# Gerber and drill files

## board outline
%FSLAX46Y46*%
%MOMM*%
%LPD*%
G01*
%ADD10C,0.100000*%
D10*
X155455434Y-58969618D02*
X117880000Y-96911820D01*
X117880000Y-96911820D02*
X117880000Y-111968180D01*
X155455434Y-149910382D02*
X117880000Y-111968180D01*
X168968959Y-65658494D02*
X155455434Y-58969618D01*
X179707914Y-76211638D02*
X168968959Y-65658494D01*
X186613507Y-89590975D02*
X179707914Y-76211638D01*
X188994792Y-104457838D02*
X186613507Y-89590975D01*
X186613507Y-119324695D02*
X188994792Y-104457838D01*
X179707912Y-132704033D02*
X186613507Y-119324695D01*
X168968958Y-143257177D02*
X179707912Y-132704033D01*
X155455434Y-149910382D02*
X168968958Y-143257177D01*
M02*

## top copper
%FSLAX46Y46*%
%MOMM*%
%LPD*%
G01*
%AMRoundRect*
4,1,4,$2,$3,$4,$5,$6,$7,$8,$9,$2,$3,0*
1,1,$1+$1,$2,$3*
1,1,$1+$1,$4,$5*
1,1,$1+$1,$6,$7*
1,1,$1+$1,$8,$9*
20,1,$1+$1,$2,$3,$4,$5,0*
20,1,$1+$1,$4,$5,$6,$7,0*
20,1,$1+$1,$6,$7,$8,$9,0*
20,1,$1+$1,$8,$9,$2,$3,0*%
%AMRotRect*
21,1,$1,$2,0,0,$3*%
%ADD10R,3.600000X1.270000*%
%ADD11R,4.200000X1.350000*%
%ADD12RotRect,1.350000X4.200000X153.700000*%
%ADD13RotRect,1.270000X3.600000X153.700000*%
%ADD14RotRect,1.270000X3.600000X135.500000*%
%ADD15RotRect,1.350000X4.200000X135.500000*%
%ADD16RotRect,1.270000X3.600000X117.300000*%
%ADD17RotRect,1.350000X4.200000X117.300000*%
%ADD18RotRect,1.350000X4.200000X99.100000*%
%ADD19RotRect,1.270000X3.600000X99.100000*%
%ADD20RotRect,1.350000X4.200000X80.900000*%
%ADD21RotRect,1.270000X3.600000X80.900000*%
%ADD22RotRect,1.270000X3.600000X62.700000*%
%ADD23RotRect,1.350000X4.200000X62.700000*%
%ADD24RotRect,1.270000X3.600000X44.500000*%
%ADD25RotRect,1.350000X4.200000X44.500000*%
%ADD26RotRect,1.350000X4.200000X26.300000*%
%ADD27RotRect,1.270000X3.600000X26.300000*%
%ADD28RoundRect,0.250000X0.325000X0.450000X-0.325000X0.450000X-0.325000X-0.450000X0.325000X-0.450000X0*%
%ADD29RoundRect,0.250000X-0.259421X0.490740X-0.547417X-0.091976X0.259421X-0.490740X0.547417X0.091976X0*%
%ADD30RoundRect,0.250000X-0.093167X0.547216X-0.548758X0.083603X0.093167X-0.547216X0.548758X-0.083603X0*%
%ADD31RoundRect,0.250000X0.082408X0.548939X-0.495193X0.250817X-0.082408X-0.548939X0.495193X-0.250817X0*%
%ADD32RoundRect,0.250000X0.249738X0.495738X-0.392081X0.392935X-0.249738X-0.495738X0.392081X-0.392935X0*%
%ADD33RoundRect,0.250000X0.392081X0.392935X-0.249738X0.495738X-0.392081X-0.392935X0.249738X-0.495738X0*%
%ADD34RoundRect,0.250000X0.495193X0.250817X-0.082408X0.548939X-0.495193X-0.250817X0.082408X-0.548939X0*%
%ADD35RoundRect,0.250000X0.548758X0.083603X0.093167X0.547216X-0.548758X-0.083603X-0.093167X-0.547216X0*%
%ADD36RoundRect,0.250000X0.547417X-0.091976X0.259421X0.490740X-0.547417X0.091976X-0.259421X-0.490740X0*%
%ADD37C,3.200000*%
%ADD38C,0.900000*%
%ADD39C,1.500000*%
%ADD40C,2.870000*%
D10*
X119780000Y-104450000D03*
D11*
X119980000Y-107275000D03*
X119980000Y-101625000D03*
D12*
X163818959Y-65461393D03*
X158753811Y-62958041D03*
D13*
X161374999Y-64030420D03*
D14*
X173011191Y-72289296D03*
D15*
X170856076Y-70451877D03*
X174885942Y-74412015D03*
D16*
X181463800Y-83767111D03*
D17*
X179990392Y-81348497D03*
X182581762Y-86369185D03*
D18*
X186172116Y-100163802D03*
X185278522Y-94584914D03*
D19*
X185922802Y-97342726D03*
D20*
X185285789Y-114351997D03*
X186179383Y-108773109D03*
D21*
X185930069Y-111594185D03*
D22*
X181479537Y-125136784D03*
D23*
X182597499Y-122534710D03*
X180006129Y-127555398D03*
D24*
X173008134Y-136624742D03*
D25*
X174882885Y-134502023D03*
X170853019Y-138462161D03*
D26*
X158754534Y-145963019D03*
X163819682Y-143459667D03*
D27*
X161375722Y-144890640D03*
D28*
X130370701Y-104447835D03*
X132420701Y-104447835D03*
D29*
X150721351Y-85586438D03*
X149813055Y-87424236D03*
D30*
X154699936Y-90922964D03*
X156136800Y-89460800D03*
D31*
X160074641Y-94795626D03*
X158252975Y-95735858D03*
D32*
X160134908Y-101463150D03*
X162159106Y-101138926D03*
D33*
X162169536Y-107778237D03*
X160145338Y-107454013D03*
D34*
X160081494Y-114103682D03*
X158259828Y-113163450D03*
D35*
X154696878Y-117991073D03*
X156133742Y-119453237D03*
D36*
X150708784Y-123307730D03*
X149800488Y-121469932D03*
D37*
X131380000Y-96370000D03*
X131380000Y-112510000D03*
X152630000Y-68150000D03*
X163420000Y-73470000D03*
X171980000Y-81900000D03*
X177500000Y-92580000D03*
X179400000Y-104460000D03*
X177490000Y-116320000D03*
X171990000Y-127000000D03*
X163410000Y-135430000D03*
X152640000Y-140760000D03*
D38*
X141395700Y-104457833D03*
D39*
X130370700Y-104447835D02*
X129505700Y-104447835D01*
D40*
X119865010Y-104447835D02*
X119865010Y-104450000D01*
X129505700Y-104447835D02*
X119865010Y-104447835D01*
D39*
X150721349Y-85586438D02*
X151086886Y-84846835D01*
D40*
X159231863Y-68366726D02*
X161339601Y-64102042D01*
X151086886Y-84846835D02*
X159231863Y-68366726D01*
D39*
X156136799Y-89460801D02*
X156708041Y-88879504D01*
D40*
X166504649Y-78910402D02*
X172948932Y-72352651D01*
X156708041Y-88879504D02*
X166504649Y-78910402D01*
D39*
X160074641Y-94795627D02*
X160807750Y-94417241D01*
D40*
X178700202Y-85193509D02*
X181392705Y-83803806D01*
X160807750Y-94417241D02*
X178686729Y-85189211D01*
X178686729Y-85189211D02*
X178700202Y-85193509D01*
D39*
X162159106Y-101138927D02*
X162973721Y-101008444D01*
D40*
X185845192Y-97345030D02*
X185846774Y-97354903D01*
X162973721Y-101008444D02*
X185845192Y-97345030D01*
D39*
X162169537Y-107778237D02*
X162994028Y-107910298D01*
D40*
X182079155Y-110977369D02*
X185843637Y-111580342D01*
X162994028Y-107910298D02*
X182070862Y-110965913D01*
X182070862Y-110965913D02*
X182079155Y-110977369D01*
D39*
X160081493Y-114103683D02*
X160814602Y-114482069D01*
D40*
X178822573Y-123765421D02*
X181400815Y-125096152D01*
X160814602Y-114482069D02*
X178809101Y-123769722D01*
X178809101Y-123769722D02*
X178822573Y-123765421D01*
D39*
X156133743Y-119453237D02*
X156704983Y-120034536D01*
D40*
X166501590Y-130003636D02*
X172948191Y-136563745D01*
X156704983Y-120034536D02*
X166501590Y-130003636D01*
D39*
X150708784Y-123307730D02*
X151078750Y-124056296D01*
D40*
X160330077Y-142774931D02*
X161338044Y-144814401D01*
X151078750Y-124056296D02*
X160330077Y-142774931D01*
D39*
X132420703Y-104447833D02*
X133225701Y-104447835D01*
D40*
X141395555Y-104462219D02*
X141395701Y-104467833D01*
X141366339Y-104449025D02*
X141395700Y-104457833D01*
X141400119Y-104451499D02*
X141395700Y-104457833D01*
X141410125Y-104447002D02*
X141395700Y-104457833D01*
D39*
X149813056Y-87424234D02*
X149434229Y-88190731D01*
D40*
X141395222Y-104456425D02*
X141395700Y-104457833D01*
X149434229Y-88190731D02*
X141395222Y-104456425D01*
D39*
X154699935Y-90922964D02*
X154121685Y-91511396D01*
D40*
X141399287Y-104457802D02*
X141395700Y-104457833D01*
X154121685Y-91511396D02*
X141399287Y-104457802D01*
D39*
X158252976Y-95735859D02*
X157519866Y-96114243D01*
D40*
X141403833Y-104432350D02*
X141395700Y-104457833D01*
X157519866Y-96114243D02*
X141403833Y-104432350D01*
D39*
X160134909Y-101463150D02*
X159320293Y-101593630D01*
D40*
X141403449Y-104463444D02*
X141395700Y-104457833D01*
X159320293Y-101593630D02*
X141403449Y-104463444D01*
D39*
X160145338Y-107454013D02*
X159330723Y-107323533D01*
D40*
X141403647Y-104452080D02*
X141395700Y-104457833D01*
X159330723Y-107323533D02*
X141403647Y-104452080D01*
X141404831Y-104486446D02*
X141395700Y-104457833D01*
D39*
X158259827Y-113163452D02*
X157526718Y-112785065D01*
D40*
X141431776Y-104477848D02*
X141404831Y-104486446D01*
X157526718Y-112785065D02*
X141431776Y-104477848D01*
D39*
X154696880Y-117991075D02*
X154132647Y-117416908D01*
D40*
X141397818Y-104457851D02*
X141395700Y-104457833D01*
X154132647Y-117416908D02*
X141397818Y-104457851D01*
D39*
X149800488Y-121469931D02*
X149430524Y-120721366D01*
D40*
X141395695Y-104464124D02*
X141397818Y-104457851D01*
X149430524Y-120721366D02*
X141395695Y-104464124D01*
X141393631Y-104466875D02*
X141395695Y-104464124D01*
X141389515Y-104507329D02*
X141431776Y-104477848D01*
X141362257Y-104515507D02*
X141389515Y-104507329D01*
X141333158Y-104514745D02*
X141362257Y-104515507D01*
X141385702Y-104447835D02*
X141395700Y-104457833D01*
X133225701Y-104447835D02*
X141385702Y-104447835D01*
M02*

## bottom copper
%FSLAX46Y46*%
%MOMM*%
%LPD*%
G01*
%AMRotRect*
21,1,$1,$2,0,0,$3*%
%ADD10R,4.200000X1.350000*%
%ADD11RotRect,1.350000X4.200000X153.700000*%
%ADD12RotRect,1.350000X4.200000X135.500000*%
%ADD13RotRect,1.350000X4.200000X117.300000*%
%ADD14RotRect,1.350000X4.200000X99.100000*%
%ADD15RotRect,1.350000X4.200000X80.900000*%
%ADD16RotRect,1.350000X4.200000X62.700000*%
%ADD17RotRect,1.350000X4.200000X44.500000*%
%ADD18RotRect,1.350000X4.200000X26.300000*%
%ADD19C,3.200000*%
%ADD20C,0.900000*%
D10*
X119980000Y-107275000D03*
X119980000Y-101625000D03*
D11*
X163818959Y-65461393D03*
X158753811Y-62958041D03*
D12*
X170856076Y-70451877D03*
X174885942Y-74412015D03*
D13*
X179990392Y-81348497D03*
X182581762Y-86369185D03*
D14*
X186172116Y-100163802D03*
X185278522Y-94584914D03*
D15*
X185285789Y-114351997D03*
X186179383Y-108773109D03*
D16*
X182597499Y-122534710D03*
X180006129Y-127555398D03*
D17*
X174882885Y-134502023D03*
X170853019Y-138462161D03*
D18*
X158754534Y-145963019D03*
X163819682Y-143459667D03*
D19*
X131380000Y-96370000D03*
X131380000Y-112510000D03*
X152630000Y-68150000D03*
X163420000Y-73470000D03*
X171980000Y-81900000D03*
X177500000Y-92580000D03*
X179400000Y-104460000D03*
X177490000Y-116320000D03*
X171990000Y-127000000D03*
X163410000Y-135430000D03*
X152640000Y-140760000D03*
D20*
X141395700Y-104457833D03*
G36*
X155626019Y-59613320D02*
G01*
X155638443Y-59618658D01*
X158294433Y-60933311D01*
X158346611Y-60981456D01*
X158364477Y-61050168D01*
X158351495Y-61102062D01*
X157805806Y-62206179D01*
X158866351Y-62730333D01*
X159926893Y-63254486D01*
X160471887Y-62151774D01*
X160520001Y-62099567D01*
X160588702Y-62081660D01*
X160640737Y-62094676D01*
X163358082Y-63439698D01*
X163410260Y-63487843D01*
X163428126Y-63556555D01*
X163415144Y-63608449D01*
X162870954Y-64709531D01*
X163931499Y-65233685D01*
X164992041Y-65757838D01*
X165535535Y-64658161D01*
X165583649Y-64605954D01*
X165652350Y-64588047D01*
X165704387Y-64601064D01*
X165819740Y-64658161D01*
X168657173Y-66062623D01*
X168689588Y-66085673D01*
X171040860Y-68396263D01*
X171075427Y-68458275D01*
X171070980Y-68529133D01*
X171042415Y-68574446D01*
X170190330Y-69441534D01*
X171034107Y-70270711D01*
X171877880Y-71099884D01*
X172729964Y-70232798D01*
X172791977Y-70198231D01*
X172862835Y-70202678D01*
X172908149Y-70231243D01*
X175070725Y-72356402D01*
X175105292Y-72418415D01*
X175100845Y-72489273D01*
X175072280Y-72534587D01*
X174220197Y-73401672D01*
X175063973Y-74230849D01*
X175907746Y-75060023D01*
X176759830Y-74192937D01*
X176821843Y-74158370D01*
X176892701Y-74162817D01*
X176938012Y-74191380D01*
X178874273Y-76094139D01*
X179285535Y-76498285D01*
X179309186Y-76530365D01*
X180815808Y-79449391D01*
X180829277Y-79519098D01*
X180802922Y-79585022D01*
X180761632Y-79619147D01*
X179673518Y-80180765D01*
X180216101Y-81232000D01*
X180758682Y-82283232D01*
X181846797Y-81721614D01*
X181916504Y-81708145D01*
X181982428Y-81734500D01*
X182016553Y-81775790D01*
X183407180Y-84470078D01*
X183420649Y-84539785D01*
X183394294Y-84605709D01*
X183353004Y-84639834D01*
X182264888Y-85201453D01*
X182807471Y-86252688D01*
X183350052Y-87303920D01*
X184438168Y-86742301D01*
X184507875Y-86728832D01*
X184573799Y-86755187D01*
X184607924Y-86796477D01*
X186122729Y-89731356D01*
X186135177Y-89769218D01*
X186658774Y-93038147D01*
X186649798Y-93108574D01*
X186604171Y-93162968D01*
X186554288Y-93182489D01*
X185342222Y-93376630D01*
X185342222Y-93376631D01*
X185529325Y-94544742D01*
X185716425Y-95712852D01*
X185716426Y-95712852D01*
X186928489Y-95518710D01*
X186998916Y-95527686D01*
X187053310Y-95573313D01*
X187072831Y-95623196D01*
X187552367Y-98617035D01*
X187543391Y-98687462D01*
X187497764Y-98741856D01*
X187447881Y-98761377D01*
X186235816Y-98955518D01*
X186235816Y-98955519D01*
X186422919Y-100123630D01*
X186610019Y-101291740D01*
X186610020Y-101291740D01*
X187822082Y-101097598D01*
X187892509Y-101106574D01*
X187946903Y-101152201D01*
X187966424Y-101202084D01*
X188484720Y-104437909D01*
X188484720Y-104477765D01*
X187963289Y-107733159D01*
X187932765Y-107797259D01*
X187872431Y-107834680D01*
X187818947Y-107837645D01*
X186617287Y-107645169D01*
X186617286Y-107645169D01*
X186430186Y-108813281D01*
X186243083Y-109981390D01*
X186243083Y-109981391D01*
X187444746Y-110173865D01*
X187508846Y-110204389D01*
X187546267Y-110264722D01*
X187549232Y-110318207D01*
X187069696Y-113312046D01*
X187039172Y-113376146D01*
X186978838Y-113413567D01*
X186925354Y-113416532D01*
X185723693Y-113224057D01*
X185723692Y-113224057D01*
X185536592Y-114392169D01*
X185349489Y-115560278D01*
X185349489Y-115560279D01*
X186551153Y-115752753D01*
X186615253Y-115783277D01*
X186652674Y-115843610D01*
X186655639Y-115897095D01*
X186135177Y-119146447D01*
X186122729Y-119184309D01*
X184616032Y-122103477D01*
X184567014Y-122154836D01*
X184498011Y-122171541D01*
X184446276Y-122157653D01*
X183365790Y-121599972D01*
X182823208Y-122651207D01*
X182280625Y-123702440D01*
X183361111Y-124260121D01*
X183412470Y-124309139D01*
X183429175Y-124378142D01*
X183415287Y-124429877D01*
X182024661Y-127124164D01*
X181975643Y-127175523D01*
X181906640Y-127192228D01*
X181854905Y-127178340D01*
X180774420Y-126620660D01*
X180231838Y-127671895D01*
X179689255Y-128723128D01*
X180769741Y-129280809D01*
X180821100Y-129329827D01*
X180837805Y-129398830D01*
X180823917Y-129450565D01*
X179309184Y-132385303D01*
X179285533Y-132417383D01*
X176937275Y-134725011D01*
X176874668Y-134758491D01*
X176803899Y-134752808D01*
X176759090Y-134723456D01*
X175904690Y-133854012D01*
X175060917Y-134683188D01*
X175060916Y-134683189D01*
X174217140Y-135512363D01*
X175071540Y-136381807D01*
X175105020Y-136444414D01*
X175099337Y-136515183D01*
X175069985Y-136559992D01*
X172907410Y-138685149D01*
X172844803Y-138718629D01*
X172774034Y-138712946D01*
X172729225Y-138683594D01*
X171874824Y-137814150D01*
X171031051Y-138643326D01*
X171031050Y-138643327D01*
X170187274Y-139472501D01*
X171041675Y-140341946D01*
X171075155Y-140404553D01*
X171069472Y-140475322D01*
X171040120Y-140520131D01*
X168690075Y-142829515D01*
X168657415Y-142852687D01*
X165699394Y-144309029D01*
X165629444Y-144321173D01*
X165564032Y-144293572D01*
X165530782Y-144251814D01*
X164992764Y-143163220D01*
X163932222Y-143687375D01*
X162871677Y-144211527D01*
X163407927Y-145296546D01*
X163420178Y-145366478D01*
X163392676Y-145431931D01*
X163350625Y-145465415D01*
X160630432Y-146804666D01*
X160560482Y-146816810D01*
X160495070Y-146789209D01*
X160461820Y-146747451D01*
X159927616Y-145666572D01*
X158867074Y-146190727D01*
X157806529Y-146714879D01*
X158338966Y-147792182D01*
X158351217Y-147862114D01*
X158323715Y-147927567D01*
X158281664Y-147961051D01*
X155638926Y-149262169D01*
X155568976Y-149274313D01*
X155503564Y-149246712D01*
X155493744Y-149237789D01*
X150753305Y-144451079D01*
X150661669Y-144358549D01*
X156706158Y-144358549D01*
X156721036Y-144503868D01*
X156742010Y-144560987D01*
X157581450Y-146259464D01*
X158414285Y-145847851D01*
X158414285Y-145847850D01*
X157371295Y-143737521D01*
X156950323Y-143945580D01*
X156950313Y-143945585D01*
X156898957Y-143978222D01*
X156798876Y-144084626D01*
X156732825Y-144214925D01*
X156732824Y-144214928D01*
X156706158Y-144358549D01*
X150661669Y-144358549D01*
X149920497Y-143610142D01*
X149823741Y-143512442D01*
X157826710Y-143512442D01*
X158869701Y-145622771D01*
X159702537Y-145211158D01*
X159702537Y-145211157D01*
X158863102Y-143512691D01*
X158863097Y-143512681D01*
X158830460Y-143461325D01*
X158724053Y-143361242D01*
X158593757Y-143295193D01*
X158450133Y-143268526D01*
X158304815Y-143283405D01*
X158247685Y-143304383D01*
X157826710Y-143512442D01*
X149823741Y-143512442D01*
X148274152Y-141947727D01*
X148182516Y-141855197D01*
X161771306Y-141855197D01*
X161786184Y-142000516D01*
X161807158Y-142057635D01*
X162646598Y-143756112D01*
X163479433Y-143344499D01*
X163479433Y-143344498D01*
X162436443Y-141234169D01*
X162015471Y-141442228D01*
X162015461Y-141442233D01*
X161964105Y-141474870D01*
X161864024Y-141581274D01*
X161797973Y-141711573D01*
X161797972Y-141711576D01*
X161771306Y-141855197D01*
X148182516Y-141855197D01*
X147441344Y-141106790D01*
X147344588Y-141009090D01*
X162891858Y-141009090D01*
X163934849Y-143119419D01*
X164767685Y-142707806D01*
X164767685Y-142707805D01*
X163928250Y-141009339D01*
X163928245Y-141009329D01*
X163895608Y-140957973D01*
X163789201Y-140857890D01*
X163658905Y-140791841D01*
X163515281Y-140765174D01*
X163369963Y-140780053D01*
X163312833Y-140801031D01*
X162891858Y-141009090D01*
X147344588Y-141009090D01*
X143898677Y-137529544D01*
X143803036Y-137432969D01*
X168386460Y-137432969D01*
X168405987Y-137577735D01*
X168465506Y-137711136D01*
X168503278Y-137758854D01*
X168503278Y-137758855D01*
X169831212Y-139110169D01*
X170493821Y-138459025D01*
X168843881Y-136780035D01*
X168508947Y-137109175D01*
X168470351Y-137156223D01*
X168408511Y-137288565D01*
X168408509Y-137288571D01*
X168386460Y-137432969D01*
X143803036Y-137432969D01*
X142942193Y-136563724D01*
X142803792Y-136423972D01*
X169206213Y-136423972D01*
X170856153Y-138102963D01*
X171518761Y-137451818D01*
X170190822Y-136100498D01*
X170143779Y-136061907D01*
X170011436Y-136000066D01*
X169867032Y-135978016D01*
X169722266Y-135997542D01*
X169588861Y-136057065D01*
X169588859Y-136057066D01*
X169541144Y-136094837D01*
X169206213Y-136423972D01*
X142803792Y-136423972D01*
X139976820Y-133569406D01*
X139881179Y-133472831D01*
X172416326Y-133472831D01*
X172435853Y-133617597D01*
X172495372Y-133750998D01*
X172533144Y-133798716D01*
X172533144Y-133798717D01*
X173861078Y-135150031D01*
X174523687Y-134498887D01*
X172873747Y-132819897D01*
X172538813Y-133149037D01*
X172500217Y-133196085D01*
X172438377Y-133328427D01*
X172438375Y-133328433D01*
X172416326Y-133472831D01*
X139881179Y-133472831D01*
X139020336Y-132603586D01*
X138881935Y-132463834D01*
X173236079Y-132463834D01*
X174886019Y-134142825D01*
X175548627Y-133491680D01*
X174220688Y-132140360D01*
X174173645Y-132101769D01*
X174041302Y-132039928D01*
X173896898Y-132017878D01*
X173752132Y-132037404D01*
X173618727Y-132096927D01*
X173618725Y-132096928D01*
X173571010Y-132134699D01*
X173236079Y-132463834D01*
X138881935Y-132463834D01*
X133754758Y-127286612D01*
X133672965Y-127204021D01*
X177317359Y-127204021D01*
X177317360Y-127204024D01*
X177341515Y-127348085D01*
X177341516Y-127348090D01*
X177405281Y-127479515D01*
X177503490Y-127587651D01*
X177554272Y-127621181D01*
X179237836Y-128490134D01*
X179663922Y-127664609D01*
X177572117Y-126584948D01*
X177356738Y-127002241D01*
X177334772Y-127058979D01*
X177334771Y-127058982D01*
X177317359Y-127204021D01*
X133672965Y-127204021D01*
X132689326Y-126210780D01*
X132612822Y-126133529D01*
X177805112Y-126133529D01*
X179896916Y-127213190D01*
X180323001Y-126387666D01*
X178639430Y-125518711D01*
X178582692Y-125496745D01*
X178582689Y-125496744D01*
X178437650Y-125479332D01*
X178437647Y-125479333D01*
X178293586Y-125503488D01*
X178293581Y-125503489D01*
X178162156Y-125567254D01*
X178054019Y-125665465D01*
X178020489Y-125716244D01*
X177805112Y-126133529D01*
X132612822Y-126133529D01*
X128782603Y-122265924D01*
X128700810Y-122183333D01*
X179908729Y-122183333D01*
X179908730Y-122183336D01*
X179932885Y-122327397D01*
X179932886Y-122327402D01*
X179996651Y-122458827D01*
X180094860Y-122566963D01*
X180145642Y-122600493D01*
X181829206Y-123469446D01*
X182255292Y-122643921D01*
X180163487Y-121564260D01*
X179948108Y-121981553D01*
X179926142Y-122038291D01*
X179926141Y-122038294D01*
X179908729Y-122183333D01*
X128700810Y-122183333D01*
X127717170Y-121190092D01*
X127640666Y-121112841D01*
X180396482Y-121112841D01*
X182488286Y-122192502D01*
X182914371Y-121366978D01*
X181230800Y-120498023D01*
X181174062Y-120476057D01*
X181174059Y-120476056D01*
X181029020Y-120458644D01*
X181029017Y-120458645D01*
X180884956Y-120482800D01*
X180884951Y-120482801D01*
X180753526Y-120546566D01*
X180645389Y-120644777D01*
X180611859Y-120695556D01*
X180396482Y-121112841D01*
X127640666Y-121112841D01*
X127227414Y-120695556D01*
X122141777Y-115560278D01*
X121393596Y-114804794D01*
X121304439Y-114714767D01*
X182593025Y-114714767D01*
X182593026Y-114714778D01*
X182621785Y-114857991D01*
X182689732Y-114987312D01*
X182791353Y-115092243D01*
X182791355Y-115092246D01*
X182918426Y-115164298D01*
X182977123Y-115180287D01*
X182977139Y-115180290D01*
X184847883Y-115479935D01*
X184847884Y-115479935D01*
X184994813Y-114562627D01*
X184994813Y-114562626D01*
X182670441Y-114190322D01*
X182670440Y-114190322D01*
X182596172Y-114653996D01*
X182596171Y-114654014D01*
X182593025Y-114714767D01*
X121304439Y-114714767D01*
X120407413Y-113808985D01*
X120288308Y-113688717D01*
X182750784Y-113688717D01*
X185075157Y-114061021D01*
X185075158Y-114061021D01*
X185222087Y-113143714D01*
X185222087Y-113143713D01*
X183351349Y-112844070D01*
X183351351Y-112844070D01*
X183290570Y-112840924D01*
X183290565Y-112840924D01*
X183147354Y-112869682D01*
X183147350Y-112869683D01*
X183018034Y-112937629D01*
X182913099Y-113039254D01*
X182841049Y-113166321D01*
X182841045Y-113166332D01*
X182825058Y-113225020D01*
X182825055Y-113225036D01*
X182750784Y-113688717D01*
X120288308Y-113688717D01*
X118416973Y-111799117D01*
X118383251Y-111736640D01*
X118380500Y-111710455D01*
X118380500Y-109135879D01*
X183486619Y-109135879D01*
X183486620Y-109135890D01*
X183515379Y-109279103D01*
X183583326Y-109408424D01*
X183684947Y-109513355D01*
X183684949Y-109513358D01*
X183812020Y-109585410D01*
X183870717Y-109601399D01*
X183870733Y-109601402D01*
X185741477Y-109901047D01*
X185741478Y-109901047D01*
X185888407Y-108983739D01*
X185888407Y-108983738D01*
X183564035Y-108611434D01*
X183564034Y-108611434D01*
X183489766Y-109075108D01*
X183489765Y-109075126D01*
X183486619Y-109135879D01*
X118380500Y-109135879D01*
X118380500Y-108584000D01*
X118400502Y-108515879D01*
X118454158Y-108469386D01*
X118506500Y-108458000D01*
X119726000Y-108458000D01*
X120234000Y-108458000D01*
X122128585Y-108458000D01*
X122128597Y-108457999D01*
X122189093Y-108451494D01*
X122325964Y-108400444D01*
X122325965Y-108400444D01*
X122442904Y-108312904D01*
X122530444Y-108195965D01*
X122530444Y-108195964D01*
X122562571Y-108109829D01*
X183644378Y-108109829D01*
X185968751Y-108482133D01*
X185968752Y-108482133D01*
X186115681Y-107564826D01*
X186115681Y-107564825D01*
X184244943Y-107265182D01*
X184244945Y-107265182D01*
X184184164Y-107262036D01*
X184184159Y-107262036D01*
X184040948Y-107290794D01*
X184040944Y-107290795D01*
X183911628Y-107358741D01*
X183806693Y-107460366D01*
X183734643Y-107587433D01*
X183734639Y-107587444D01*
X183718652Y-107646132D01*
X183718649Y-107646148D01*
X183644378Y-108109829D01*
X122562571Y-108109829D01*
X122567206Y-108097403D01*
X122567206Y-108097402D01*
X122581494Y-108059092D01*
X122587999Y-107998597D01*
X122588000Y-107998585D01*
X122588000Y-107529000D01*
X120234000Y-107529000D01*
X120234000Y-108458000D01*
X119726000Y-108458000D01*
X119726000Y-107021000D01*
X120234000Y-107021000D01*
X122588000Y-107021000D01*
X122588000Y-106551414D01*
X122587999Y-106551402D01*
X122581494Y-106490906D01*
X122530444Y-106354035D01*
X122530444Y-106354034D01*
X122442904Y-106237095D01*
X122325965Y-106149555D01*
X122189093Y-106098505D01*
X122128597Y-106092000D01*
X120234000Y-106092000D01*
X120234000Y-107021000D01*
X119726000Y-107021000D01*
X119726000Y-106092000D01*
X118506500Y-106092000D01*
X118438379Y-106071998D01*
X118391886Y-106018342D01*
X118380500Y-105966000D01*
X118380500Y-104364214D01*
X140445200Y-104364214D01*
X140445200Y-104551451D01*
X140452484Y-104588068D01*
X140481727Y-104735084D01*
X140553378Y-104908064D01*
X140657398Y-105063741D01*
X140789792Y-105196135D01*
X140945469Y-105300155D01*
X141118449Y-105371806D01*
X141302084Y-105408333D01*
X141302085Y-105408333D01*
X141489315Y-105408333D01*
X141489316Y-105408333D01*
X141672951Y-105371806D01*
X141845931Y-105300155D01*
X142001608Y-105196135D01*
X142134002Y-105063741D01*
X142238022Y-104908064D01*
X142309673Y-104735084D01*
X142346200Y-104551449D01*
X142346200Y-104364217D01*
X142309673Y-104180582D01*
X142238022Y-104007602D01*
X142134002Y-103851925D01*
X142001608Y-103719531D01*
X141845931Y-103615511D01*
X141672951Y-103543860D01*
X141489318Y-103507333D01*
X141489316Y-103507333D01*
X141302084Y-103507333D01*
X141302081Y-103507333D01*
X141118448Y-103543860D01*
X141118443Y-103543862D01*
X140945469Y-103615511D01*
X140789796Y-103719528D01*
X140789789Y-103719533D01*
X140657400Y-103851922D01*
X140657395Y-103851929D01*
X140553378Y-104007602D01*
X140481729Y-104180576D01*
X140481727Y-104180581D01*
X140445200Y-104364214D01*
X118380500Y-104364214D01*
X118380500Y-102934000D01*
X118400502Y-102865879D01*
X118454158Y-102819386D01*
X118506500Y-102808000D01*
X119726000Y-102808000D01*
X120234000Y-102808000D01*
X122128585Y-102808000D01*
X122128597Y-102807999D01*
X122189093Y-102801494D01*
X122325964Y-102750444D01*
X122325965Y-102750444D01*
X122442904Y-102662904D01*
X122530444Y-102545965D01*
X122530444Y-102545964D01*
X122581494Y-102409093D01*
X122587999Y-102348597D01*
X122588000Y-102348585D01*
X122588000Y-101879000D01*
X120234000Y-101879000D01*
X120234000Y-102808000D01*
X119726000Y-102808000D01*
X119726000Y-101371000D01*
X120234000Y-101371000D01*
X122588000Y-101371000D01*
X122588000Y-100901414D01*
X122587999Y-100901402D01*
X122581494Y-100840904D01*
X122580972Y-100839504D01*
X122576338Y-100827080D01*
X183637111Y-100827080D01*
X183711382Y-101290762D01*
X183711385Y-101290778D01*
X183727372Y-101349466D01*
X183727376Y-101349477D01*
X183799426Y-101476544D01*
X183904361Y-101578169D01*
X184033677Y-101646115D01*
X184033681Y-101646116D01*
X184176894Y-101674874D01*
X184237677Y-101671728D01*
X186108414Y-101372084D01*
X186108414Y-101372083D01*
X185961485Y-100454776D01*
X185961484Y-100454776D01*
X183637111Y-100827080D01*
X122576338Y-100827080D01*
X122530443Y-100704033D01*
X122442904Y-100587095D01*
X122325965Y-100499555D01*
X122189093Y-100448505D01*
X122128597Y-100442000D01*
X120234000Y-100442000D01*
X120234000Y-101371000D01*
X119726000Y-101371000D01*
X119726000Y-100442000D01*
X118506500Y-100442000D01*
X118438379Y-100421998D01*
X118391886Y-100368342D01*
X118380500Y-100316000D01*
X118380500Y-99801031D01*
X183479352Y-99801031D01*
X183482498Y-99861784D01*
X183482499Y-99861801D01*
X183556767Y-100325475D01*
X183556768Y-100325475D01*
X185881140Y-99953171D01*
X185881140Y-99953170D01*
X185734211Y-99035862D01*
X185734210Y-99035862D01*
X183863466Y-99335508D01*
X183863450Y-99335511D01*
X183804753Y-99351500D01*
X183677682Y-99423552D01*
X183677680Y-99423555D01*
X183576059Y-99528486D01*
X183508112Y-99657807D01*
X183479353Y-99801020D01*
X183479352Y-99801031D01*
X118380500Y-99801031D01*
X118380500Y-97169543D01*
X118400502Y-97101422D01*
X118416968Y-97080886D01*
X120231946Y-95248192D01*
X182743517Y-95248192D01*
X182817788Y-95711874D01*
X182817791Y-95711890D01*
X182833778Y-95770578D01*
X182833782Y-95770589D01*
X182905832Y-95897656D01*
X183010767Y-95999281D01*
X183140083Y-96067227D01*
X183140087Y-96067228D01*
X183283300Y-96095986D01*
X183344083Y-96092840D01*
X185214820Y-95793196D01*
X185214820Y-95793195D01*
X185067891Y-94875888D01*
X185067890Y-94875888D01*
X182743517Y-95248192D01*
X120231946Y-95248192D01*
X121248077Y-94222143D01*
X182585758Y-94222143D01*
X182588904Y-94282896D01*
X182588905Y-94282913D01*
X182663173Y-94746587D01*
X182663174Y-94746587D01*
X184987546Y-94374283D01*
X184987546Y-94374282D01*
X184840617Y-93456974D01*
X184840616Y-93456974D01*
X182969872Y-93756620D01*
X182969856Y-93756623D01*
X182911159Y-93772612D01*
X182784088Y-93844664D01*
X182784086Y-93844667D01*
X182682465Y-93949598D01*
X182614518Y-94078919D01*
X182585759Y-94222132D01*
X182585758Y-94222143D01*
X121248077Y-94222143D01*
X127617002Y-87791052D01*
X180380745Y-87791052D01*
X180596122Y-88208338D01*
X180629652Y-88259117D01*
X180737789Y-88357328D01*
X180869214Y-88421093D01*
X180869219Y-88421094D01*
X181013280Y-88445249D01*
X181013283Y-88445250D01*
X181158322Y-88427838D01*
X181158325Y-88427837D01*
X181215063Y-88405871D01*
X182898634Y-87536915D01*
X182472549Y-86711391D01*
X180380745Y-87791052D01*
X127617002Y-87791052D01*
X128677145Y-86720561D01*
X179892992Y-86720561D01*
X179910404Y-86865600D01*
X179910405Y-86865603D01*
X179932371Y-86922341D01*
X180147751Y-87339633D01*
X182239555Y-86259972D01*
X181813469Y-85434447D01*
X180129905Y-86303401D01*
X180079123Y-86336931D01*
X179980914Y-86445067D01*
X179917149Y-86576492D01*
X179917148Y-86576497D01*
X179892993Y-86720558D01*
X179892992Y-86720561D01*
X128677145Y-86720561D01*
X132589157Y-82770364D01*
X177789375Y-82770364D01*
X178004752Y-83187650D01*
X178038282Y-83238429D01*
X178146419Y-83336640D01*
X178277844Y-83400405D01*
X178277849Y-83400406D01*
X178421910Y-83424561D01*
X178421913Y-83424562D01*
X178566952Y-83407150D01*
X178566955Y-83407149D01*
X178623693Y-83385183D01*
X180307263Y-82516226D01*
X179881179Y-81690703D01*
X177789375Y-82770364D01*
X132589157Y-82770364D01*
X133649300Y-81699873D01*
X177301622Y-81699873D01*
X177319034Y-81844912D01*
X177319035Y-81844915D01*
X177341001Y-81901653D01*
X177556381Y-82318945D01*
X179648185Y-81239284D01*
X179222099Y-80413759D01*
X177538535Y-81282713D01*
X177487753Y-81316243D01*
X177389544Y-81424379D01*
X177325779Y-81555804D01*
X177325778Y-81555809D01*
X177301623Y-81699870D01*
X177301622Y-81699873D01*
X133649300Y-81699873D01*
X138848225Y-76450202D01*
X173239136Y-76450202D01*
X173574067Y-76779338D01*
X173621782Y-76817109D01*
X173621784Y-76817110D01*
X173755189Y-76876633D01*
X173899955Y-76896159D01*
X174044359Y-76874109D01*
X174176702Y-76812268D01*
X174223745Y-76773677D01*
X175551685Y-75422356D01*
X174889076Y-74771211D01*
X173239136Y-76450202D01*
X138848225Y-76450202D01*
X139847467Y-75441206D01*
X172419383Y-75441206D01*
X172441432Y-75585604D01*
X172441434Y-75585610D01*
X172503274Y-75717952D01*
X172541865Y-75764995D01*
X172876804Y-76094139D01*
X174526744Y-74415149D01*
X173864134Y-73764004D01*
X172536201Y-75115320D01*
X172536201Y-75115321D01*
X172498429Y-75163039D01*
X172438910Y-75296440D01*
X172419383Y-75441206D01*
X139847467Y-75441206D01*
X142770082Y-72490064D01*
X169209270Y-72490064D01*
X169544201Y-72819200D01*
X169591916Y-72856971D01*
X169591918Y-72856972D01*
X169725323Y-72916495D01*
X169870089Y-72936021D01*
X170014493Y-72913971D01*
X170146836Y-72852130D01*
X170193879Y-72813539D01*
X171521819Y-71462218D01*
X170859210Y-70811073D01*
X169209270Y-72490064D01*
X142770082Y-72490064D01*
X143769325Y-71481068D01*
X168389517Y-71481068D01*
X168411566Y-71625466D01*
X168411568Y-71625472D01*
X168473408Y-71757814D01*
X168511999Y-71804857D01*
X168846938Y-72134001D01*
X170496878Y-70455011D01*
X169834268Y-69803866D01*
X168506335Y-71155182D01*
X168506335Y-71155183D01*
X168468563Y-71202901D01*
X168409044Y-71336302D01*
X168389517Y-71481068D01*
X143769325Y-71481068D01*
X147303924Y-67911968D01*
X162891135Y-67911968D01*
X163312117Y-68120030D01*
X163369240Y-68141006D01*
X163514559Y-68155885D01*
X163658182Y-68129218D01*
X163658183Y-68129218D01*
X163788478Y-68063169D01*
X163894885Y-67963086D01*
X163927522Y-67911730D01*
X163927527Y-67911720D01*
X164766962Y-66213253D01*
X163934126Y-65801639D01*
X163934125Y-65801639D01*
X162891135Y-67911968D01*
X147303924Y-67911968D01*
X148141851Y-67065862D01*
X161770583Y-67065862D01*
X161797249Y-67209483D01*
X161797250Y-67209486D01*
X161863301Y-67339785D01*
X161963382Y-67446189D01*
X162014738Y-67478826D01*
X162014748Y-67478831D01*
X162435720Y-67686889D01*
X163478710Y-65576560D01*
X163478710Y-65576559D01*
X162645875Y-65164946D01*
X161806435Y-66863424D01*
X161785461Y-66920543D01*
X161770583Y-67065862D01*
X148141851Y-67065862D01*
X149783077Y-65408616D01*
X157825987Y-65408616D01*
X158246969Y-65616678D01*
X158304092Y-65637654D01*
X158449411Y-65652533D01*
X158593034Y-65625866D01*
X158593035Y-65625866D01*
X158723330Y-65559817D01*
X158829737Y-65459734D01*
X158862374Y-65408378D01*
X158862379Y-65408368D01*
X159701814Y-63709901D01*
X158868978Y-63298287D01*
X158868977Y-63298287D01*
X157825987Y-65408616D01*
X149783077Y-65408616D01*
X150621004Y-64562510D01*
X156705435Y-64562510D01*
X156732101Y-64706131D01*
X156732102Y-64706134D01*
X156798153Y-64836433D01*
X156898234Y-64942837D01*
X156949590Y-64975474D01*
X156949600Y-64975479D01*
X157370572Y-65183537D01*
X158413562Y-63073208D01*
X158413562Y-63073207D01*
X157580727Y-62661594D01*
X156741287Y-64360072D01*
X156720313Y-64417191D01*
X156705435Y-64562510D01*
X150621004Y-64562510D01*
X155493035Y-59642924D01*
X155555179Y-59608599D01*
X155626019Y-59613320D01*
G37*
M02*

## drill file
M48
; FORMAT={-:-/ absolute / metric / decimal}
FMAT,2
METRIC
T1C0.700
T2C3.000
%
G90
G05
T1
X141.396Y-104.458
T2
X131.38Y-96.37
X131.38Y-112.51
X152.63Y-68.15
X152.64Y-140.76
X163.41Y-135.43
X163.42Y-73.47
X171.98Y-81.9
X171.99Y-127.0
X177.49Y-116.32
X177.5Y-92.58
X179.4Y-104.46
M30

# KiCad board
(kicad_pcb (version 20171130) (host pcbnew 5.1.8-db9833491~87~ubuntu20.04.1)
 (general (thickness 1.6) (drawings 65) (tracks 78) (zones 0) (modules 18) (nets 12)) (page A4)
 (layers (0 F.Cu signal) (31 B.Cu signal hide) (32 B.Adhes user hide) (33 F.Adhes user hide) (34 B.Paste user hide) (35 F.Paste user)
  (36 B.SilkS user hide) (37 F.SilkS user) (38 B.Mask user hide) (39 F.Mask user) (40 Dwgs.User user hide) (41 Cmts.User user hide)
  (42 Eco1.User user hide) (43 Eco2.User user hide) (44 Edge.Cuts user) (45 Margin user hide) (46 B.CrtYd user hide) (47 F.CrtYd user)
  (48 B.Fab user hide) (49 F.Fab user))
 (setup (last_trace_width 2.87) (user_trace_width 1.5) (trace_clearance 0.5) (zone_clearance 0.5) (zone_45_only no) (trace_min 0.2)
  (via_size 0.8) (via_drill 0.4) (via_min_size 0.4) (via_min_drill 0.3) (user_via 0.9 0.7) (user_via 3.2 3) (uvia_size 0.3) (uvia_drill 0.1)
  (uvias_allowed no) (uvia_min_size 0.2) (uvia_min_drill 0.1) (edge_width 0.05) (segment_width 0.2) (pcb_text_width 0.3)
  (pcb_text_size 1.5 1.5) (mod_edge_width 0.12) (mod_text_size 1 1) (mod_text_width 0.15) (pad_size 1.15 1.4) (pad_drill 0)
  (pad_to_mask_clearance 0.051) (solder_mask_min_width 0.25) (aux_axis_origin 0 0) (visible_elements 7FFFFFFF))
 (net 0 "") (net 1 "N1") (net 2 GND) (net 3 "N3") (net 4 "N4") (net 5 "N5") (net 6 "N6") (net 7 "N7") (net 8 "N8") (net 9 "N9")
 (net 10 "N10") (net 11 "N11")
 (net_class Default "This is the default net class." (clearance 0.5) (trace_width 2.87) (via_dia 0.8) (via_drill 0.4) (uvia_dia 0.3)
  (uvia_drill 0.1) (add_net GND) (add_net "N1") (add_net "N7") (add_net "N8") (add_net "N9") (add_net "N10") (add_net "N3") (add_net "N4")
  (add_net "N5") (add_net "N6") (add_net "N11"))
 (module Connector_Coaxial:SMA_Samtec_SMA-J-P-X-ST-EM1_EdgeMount (layer F.Cu) (at 119.98 104.45 270)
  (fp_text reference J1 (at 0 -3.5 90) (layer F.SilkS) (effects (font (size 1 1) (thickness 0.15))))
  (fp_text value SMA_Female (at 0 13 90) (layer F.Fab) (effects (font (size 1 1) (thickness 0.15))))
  (pad 1 smd rect (at 0 0.2 270) (size 1.27 3.6) (layers F.Cu F.Paste F.Mask) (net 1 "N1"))
  (pad 2 smd rect (at 2.825 0 270) (size 1.35 4.2) (layers F.Cu F.Paste F.Mask) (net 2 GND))
  (pad 2 smd rect (at -2.825 0 270) (size 1.35 4.2) (layers F.Cu F.Paste F.Mask) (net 2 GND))
  (pad 2 smd rect (at 2.825 0 270) (size 1.35 4.2) (layers B.Cu B.Paste B.Mask) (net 2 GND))
  (pad 2 smd rect (at -2.825 0 270) (size 1.35 4.2) (layers B.Cu B.Paste B.Mask) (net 2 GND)))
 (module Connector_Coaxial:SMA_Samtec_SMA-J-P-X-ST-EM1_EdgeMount (layer F.Cu) (at 161.286385 64.209717 153.7)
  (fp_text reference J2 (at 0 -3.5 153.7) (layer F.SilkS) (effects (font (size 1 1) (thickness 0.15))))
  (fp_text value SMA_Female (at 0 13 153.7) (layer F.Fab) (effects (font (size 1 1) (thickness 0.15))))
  (pad 2 smd rect (at -2.825 0 153.7) (size 1.35 4.2) (layers B.Cu B.Paste B.Mask) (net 2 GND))
  (pad 2 smd rect (at 2.825 0 153.7) (size 1.35 4.2) (layers B.Cu B.Paste B.Mask) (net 2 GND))
  (pad 2 smd rect (at -2.825 0 153.7) (size 1.35 4.2) (layers F.Cu F.Paste F.Mask) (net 2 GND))
  (pad 2 smd rect (at 2.825 0 153.7) (size 1.35 4.2) (layers F.Cu F.Paste F.Mask) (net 2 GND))
  (pad 1 smd rect (at 0 0.2 153.7) (size 1.27 3.6) (layers F.Cu F.Paste F.Mask) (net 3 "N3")))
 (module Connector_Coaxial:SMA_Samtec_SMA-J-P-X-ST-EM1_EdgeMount (layer F.Cu) (at 172.871009 72.431946 135.5)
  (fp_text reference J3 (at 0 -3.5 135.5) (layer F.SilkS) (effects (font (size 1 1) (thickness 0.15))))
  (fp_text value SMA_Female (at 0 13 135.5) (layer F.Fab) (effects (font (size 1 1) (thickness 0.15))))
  (pad 1 smd rect (at 0 0.2 135.5) (size 1.27 3.6) (layers F.Cu F.Paste F.Mask) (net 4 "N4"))
  (pad 2 smd rect (at 2.825 0 135.5) (size 1.35 4.2) (layers F.Cu F.Paste F.Mask) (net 2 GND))
  (pad 2 smd rect (at -2.825 0 135.5) (size 1.35 4.2) (layers F.Cu F.Paste F.Mask) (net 2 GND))
  (pad 2 smd rect (at 2.825 0 135.5) (size 1.35 4.2) (layers B.Cu B.Paste B.Mask) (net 2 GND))
  (pad 2 smd rect (at -2.825 0 135.5) (size 1.35 4.2) (layers B.Cu B.Paste B.Mask) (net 2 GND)))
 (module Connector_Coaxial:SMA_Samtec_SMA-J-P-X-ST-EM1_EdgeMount (layer F.Cu) (at 181.286077 83.858841 117.3)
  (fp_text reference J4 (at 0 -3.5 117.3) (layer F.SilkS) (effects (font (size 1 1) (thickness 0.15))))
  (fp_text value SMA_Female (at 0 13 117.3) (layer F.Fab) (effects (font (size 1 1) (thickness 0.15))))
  (pad 1 smd rect (at 0 0.2 117.3) (size 1.27 3.6) (layers F.Cu F.Paste F.Mask) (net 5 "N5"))
  (pad 2 smd rect (at 2.825 0 117.3) (size 1.35 4.2) (layers F.Cu F.Paste F.Mask) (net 2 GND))
  (pad 2 smd rect (at -2.825 0 117.3) (size 1.35 4.2) (layers F.Cu F.Paste F.Mask) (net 2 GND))
  (pad 2 smd rect (at 2.825 0 117.3) (size 1.35 4.2) (layers B.Cu B.Paste B.Mask) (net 2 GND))
  (pad 2 smd rect (at -2.825 0 117.3) (size 1.35 4.2) (layers B.Cu B.Paste B.Mask) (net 2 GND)))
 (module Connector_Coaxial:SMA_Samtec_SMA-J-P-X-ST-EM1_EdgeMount (layer F.Cu) (at 185.725319 97.374358 99.1)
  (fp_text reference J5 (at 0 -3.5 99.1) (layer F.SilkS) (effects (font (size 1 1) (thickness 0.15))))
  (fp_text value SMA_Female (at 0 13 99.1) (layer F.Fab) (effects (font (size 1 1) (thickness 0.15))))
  (pad 2 smd rect (at -2.825 0 99.1) (size 1.35 4.2) (layers B.Cu B.Paste B.Mask) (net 2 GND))
  (pad 2 smd rect (at 2.825 0 99.1) (size 1.35 4.2) (layers B.Cu B.Paste B.Mask) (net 2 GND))
  (pad 2 smd rect (at -2.825 0 99.1) (size 1.35 4.2) (layers F.Cu F.Paste F.Mask) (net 2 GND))
  (pad 2 smd rect (at 2.825 0 99.1) (size 1.35 4.2) (layers F.Cu F.Paste F.Mask) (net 2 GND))
  (pad 1 smd rect (at 0 0.2 99.1) (size 1.27 3.6) (layers F.Cu F.Paste F.Mask) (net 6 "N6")))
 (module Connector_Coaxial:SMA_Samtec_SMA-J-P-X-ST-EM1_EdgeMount (layer F.Cu) (at 185.732586 111.562553 80.9)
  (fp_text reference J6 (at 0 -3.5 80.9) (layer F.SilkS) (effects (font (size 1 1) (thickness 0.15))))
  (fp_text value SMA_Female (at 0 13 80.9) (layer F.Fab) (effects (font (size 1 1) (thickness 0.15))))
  (pad 2 smd rect (at -2.825 0 80.9) (size 1.35 4.2) (layers B.Cu B.Paste B.Mask) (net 2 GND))
  (pad 2 smd rect (at 2.825 0 80.9) (size 1.35 4.2) (layers B.Cu B.Paste B.Mask) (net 2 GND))
  (pad 2 smd rect (at -2.825 0 80.9) (size 1.35 4.2) (layers F.Cu F.Paste F.Mask) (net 2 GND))
  (pad 2 smd rect (at 2.825 0 80.9) (size 1.35 4.2) (layers F.Cu F.Paste F.Mask) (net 2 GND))
  (pad 1 smd rect (at 0 0.2 80.9) (size 1.27 3.6) (layers F.Cu F.Paste F.Mask) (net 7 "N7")))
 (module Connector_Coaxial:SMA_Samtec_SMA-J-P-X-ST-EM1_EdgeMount (layer F.Cu) (at 181.301814 125.045054 62.7)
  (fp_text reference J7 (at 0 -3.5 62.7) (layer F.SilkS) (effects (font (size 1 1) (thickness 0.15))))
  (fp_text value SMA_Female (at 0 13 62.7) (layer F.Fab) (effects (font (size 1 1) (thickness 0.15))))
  (pad 1 smd rect (at 0 0.2 62.7) (size 1.27 3.6) (layers F.Cu F.Paste F.Mask) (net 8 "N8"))
  (pad 2 smd rect (at 2.825 0 62.7) (size 1.35 4.2) (layers F.Cu F.Paste F.Mask) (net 2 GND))
  (pad 2 smd rect (at -2.825 0 62.7) (size 1.35 4.2) (layers F.Cu F.Paste F.Mask) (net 2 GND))
  (pad 2 smd rect (at 2.825 0 62.7) (size 1.35 4.2) (layers B.Cu B.Paste B.Mask) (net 2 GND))
  (pad 2 smd rect (at -2.825 0 62.7) (size 1.35 4.2) (layers B.Cu B.Paste B.Mask) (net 2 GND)))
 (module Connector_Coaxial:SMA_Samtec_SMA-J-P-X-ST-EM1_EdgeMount (layer F.Cu) (at 172.867952 136.482092 44.5)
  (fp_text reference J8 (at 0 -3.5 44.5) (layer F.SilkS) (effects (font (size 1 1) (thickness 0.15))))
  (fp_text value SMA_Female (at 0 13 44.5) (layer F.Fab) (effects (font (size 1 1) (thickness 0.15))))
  (pad 1 smd rect (at 0 0.2 44.5) (size 1.27 3.6) (layers F.Cu F.Paste F.Mask) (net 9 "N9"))
  (pad 2 smd rect (at 2.825 0 44.5) (size 1.35 4.2) (layers F.Cu F.Paste F.Mask) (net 2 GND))
  (pad 2 smd rect (at -2.825 0 44.5) (size 1.35 4.2) (layers F.Cu F.Paste F.Mask) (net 2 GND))
  (pad 2 smd rect (at 2.825 0 44.5) (size 1.35 4.2) (layers B.Cu B.Paste B.Mask) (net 2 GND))
  (pad 2 smd rect (at -2.825 0 44.5) (size 1.35 4.2) (layers B.Cu B.Paste B.Mask) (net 2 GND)))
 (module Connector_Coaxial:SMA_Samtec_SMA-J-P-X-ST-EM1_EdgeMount (layer F.Cu) (at 161.287108 144.711343 26.3)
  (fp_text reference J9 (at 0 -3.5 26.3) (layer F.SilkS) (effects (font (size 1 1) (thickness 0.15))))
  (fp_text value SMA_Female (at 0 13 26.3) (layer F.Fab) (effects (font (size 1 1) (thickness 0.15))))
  (pad 2 smd rect (at -2.825 0 26.3) (size 1.35 4.2) (layers B.Cu B.Paste B.Mask) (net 2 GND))
  (pad 2 smd rect (at 2.825 0 26.3) (size 1.35 4.2) (layers B.Cu B.Paste B.Mask) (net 2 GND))
  (pad 2 smd rect (at -2.825 0 26.3) (size 1.35 4.2) (layers F.Cu F.Paste F.Mask) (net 2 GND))
  (pad 2 smd rect (at 2.825 0 26.3) (size 1.35 4.2) (layers F.Cu F.Paste F.Mask) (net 2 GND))
  (pad 1 smd rect (at 0 0.2 26.3) (size 1.27 3.6) (layers F.Cu F.Paste F.Mask) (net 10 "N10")))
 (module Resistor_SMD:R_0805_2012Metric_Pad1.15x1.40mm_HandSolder (layer F.Cu) (at 131.395701 104.447835 180)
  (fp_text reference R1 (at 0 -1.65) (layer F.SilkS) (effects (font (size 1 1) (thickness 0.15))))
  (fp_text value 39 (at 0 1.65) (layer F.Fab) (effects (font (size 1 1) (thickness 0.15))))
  (pad 2 smd roundrect (at 1.025 0 180) (size 1.15 1.4) (layers F.Cu F.Paste F.Mask) (roundrect_rratio 0.217391) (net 1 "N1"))
  (pad 1 smd roundrect (at -1.025 0 180) (size 1.15 1.4) (layers F.Cu F.Paste F.Mask) (roundrect_rratio 0.217391) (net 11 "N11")))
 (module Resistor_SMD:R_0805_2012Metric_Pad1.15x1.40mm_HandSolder (layer F.Cu) (at 150.267203 86.505337 243.7)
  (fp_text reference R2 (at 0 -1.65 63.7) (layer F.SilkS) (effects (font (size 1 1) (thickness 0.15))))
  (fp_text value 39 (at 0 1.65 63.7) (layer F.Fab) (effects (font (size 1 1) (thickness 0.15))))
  (pad 1 smd roundrect (at -1.025 0 243.7) (size 1.15 1.4) (layers F.Cu F.Paste F.Mask) (roundrect_rratio 0.217391) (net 3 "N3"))
  (pad 2 smd roundrect (at 1.025 0 243.7) (size 1.15 1.4) (layers F.Cu F.Paste F.Mask) (roundrect_rratio 0.217391) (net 11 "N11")))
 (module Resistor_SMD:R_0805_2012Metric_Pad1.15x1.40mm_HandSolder (layer F.Cu) (at 155.418368 90.191882 225.5)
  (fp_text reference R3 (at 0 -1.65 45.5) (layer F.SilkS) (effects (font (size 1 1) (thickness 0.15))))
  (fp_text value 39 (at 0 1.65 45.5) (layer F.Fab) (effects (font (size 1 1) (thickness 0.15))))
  (pad 2 smd roundrect (at 1.025 0 225.5) (size 1.15 1.4) (layers F.Cu F.Paste F.Mask) (roundrect_rratio 0.217391) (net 11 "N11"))
  (pad 1 smd roundrect (at -1.025 0 225.5) (size 1.15 1.4) (layers F.Cu F.Paste F.Mask) (roundrect_rratio 0.217391) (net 4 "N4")))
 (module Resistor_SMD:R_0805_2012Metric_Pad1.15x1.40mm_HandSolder (layer F.Cu) (at 159.163808 95.265742 207.3)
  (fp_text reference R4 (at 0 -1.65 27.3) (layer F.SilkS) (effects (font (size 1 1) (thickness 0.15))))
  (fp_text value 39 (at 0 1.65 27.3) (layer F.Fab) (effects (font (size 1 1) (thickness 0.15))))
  (pad 1 smd roundrect (at -1.025 0 207.3) (size 1.15 1.4) (layers F.Cu F.Paste F.Mask) (roundrect_rratio 0.217391) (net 5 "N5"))
  (pad 2 smd roundrect (at 1.025 0 207.3) (size 1.15 1.4) (layers F.Cu F.Paste F.Mask) (roundrect_rratio 0.217391) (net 11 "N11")))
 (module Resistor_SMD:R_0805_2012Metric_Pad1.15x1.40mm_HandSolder (layer F.Cu) (at 161.147007 101.301038 189.1)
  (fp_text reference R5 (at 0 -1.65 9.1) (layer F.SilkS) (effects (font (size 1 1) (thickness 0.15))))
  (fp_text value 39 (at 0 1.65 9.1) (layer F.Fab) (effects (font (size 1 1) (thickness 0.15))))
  (pad 2 smd roundrect (at 1.025 0 189.1) (size 1.15 1.4) (layers F.Cu F.Paste F.Mask) (roundrect_rratio 0.217391) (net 11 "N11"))
  (pad 1 smd roundrect (at -1.025 0 189.1) (size 1.15 1.4) (layers F.Cu F.Paste F.Mask) (roundrect_rratio 0.217391) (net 6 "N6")))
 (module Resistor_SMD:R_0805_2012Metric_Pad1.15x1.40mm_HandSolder (layer F.Cu) (at 161.157437 107.616125 170.9)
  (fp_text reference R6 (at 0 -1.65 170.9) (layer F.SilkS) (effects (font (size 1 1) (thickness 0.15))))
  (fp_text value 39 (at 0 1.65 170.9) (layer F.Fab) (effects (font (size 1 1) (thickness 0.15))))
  (pad 1 smd roundrect (at -1.025 0 170.9) (size 1.15 1.4) (layers F.Cu F.Paste F.Mask) (roundrect_rratio 0.217391) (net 7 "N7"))
  (pad 2 smd roundrect (at 1.025 0 170.9) (size 1.15 1.4) (layers F.Cu F.Paste F.Mask) (roundrect_rratio 0.217391) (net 11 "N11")))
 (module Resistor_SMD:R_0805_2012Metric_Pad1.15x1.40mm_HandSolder (layer F.Cu) (at 159.170661 113.633566 152.7)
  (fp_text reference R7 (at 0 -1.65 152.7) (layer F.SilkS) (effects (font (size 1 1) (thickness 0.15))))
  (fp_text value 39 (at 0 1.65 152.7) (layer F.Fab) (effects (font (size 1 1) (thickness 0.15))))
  (pad 1 smd roundrect (at -1.025 0 152.7) (size 1.15 1.4) (layers F.Cu F.Paste F.Mask) (roundrect_rratio 0.217391) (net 8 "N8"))
  (pad 2 smd roundrect (at 1.025 0 152.7) (size 1.15 1.4) (layers F.Cu F.Paste F.Mask) (roundrect_rratio 0.217391) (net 11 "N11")))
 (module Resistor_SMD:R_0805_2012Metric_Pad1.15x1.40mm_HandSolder (layer F.Cu) (at 155.41531 118.722155 134.5)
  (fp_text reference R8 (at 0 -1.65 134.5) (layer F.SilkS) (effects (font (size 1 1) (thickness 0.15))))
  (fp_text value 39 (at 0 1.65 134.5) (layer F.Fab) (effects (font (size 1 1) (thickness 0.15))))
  (pad 2 smd roundrect (at 1.025 0 134.5) (size 1.15 1.4) (layers F.Cu F.Paste F.Mask) (roundrect_rratio 0.217391) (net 11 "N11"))
  (pad 1 smd roundrect (at -1.025 0 134.5) (size 1.15 1.4) (layers F.Cu F.Paste F.Mask) (roundrect_rratio 0.217391) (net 9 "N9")))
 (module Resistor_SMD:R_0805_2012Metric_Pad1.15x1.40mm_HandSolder (layer F.Cu) (at 150.254636 122.388831 116.3)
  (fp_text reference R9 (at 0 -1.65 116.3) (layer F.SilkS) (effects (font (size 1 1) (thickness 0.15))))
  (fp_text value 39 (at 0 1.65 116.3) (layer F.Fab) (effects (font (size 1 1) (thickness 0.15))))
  (pad 1 smd roundrect (at -1.025 0 116.3) (size 1.15 1.4) (layers F.Cu F.Paste F.Mask) (roundrect_rratio 0.217391) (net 10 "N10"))
  (pad 2 smd roundrect (at 1.025 0 116.3) (size 1.15 1.4) (layers F.Cu F.Paste F.Mask) (roundrect_rratio 0.217391) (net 11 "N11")))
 (gr_line (start 155.455434 58.969618) (end 117.88 96.91182) (layer Edge.Cuts) (width 0.1))
 (gr_line (start 117.88 96.91182) (end 117.88 111.96818) (layer Edge.Cuts) (width 0.1))
 (gr_line (start 155.455434 149.910382) (end 117.88 111.96818) (layer Edge.Cuts) (width 0.1))
 (gr_line (start 168.968959 65.658494) (end 155.455434 58.969618) (layer Edge.Cuts) (width 0.1))
 (gr_line (start 179.707914 76.211638) (end 168.968959 65.658494) (layer Edge.Cuts) (width 0.1))
 (gr_line (start 186.613507 89.590975) (end 179.707914 76.211638) (layer Edge.Cuts) (width 0.1))
 (gr_line (start 188.994792 104.457838) (end 186.613507 89.590975) (layer Edge.Cuts) (width 0.1))
 (gr_line (start 186.613507 119.324695) (end 188.994792 104.457838) (layer Edge.Cuts) (width 0.1))
 (gr_line (start 179.707912 132.704033) (end 186.613507 119.324695) (layer Edge.Cuts) (width 0.1))
 (gr_line (start 168.968958 143.257177) (end 179.707912 132.704033) (layer Edge.Cuts) (width 0.1))
 (gr_line (start 155.455434 149.910382) (end 168.968958 143.257177) (layer Edge.Cuts) (width 0.1))
 (segment (start 130.3707 104.447835) (end 129.5057 104.447835) (width 1.5) (layer F.Cu) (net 1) (status 10))
 (segment (start 119.86501 104.447835) (end 119.86501 104.45) (width 2.87) (layer F.Cu) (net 1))
 (segment (start 129.5057 104.447835) (end 119.86501 104.447835) (width 2.87) (layer F.Cu) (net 1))
 (via (at 131.38 96.37) (size 3.2) (drill 3) (layers F.Cu B.Cu) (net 2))
 (via (at 131.38 112.51) (size 3.2) (drill 3) (layers F.Cu B.Cu) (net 2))
 (via (at 152.63 68.15) (size 3.2) (drill 3) (layers F.Cu B.Cu) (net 2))
 (via (at 163.42 73.47) (size 3.2) (drill 3) (layers F.Cu B.Cu) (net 2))
 (via (at 171.98 81.9) (size 3.2) (drill 3) (layers F.Cu B.Cu) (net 2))
 (via (at 177.5 92.58) (size 3.2) (drill 3) (layers F.Cu B.Cu) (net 2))
 (via (at 179.4 104.46) (size 3.2) (drill 3) (layers F.Cu B.Cu) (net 2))
 (via (at 177.49 116.32) (size 3.2) (drill 3) (layers F.Cu B.Cu) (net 2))
 (via (at 171.99 127) (size 3.2) (drill 3) (layers F.Cu B.Cu) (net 2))
 (via (at 163.41 135.43) (size 3.2) (drill 3) (layers F.Cu B.Cu) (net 2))
 (via (at 152.64 140.76) (size 3.2) (drill 3) (layers F.Cu B.Cu) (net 2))
 (segment (start 150.721349 85.586438) (end 151.086886 84.846835) (width 1.5) (layer F.Cu) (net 3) (status 10))
 (segment (start 159.231863 68.366726) (end 161.339601 64.102042) (width 2.87) (layer F.Cu) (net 3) (status 20))
 (segment (start 151.086886 84.846835) (end 159.231863 68.366726) (width 2.87) (layer F.Cu) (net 3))
 (segment (start 156.136799 89.460801) (end 156.708041 88.879504) (width 1.5) (layer F.Cu) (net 4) (status 10))
 (segment (start 166.504649 78.910402) (end 172.948932 72.352651) (width 2.87) (layer F.Cu) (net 4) (status 20))
 (segment (start 156.708041 88.879504) (end 166.504649 78.910402) (width 2.87) (layer F.Cu) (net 4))
 (segment (start 160.074641 94.795627) (end 160.80775 94.417241) (width 1.5) (layer F.Cu) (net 5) (status 10))
 (segment (start 178.700202 85.193509) (end 181.392705 83.803806) (width 2.87) (layer F.Cu) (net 5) (status 20))
 (segment (start 160.80775 94.417241) (end 178.686729 85.189211) (width 2.87) (layer F.Cu) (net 5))
 (segment (start 178.686729 85.189211) (end 178.700202 85.193509) (width 2.87) (layer F.Cu) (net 5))
 (segment (start 162.159106 101.138927) (end 162.973721 101.008444) (width 1.5) (layer F.Cu) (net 6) (status 10))
 (segment (start 185.845192 97.34503) (end 185.846774 97.354903) (width 2.87) (layer F.Cu) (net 6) (status 30))
 (segment (start 162.973721 101.008444) (end 185.845192 97.34503) (width 2.87) (layer F.Cu) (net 6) (status 20))
 (segment (start 162.169537 107.778237) (end 162.994028 107.910298) (width 1.5) (layer F.Cu) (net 7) (status 10))
 (segment (start 182.079155 110.977369) (end 185.843637 111.580342) (width 2.87) (layer F.Cu) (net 7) (status 20))
 (segment (start 162.994028 107.910298) (end 182.070862 110.965913) (width 2.87) (layer F.Cu) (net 7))
 (segment (start 182.070862 110.965913) (end 182.079155 110.977369) (width 2.87) (layer F.Cu) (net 7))
 (segment (start 160.081493 114.103683) (end 160.814602 114.482069) (width 1.5) (layer F.Cu) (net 8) (status 10))
 (segment (start 178.822573 123.765421) (end 181.400815 125.096152) (width 2.87) (layer F.Cu) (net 8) (status 20))
 (segment (start 160.814602 114.482069) (end 178.809101 123.769722) (width 2.87) (layer F.Cu) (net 8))
 (segment (start 178.809101 123.769722) (end 178.822573 123.765421) (width 2.87) (layer F.Cu) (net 8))
 (segment (start 156.133743 119.453237) (end 156.704983 120.034536) (width 1.5) (layer F.Cu) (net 9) (status 10))
 (segment (start 166.50159 130.003636) (end 172.948191 136.563745) (width 2.87) (layer F.Cu) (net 9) (status 20))
 (segment (start 156.704983 120.034536) (end 166.50159 130.003636) (width 2.87) (layer F.Cu) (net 9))
 (segment (start 150.708784 123.30773) (end 151.07875 124.056296) (width 1.5) (layer F.Cu) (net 10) (status 10))
 (segment (start 160.330077 142.774931) (end 161.338044 144.814401) (width 2.87) (layer F.Cu) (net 10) (status 20))
 (segment (start 151.07875 124.056296) (end 160.330077 142.774931) (width 2.87) (layer F.Cu) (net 10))
 (via (at 141.3957 104.457833) (size 0.9) (drill 0.7) (layers F.Cu B.Cu) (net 11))
 (segment (start 132.420703 104.447833) (end 133.225701 104.447835) (width 1.5) (layer F.Cu) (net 11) (status 10))
 (segment (start 141.395555 104.462219) (end 141.395701 104.467833) (width 2.87) (layer F.Cu) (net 11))
 (segment (start 141.366339 104.449025) (end 141.3957 104.457833) (width 2.87) (layer F.Cu) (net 11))
 (segment (start 141.400119 104.451499) (end 141.3957 104.457833) (width 2.87) (layer F.Cu) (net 11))
 (segment (start 141.410125 104.447002) (end 141.3957 104.457833) (width 2.87) (layer F.Cu) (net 11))
 (segment (start 149.813056 87.424234) (end 149.434229 88.190731) (width 1.5) (layer F.Cu) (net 11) (status 10))
 (segment (start 141.395222 104.456425) (end 141.3957 104.457833) (width 2.87) (layer F.Cu) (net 11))
 (segment (start 149.434229 88.190731) (end 141.395222 104.456425) (width 2.87) (layer F.Cu) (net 11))
 (segment (start 154.699935 90.922964) (end 154.121685 91.511396) (width 1.5) (layer F.Cu) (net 11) (status 10))
 (segment (start 141.399287 104.457802) (end 141.3957 104.457833) (width 2.87) (layer F.Cu) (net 11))
 (segment (start 154.121685 91.511396) (end 141.399287 104.457802) (width 2.87) (layer F.Cu) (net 11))
 (segment (start 158.252976 95.735859) (end 157.519866 96.114243) (width 1.5) (layer F.Cu) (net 11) (status 10))
 (segment (start 141.403833 104.43235) (end 141.3957 104.457833) (width 2.87) (layer F.Cu) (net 11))
 (segment (start 157.519866 96.114243) (end 141.403833 104.43235) (width 2.87) (layer F.Cu) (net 11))
 (segment (start 160.134909 101.46315) (end 159.320293 101.59363) (width 1.5) (layer F.Cu) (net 11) (status 10))
 (segment (start 141.403449 104.463444) (end 141.3957 104.457833) (width 2.87) (layer F.Cu) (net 11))
 (segment (start 159.320293 101.59363) (end 141.403449 104.463444) (width 2.87) (layer F.Cu) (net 11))
 (segment (start 160.145338 107.454013) (end 159.330723 107.323533) (width 1.5) (layer F.Cu) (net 11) (status 10))
 (segment (start 141.403647 104.45208) (end 141.3957 104.457833) (width 2.87) (layer F.Cu) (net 11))
 (segment (start 159.330723 107.323533) (end 141.403647 104.45208) (width 2.87) (layer F.Cu) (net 11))
 (segment (start 141.404831 104.486446) (end 141.3957 104.457833) (width 2.87) (layer F.Cu) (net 11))
 (segment (start 158.259827 113.163452) (end 157.526718 112.785065) (width 1.5) (layer F.Cu) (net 11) (status 10))
 (segment (start 141.431776 104.477848) (end 141.404831 104.486446) (width 2.87) (layer F.Cu) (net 11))
 (segment (start 157.526718 112.785065) (end 141.431776 104.477848) (width 2.87) (layer F.Cu) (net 11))
 (segment (start 154.69688 117.991075) (end 154.132647 117.416908) (width 1.5) (layer F.Cu) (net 11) (status 10))
 (segment (start 141.397818 104.457851) (end 141.3957 104.457833) (width 2.87) (layer F.Cu) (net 11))
 (segment (start 154.132647 117.416908) (end 141.397818 104.457851) (width 2.87) (layer F.Cu) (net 11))
 (segment (start 149.800488 121.469931) (end 149.430524 120.721366) (width 1.5) (layer F.Cu) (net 11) (status 10))
 (segment (start 141.395695 104.464124) (end 141.397818 104.457851) (width 2.87) (layer F.Cu) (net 11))
 (segment (start 149.430524 120.721366) (end 141.395695 104.464124) (width 2.87) (layer F.Cu) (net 11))
 (segment (start 141.393631 104.466875) (end 141.395695 104.464124) (width 2.87) (layer F.Cu) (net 11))
 (segment (start 141.389515 104.507329) (end 141.431776 104.477848) (width 2.87) (layer F.Cu) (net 11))
 (segment (start 141.362257 104.515507) (end 141.389515 104.507329) (width 2.87) (layer F.Cu) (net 11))
 (segment (start 141.333158 104.514745) (end 141.362257 104.515507) (width 2.87) (layer F.Cu) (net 11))
 (segment (start 141.385702 104.447835) (end 141.3957 104.457833) (width 2.87) (layer F.Cu) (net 11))
 (segment (start 133.225701 104.447835) (end 141.385702 104.447835) (width 2.87) (layer F.Cu) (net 11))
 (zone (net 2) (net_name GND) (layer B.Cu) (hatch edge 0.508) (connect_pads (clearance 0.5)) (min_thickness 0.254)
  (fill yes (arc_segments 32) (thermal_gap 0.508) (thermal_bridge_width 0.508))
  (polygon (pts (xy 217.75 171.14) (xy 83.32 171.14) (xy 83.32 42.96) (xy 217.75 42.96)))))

